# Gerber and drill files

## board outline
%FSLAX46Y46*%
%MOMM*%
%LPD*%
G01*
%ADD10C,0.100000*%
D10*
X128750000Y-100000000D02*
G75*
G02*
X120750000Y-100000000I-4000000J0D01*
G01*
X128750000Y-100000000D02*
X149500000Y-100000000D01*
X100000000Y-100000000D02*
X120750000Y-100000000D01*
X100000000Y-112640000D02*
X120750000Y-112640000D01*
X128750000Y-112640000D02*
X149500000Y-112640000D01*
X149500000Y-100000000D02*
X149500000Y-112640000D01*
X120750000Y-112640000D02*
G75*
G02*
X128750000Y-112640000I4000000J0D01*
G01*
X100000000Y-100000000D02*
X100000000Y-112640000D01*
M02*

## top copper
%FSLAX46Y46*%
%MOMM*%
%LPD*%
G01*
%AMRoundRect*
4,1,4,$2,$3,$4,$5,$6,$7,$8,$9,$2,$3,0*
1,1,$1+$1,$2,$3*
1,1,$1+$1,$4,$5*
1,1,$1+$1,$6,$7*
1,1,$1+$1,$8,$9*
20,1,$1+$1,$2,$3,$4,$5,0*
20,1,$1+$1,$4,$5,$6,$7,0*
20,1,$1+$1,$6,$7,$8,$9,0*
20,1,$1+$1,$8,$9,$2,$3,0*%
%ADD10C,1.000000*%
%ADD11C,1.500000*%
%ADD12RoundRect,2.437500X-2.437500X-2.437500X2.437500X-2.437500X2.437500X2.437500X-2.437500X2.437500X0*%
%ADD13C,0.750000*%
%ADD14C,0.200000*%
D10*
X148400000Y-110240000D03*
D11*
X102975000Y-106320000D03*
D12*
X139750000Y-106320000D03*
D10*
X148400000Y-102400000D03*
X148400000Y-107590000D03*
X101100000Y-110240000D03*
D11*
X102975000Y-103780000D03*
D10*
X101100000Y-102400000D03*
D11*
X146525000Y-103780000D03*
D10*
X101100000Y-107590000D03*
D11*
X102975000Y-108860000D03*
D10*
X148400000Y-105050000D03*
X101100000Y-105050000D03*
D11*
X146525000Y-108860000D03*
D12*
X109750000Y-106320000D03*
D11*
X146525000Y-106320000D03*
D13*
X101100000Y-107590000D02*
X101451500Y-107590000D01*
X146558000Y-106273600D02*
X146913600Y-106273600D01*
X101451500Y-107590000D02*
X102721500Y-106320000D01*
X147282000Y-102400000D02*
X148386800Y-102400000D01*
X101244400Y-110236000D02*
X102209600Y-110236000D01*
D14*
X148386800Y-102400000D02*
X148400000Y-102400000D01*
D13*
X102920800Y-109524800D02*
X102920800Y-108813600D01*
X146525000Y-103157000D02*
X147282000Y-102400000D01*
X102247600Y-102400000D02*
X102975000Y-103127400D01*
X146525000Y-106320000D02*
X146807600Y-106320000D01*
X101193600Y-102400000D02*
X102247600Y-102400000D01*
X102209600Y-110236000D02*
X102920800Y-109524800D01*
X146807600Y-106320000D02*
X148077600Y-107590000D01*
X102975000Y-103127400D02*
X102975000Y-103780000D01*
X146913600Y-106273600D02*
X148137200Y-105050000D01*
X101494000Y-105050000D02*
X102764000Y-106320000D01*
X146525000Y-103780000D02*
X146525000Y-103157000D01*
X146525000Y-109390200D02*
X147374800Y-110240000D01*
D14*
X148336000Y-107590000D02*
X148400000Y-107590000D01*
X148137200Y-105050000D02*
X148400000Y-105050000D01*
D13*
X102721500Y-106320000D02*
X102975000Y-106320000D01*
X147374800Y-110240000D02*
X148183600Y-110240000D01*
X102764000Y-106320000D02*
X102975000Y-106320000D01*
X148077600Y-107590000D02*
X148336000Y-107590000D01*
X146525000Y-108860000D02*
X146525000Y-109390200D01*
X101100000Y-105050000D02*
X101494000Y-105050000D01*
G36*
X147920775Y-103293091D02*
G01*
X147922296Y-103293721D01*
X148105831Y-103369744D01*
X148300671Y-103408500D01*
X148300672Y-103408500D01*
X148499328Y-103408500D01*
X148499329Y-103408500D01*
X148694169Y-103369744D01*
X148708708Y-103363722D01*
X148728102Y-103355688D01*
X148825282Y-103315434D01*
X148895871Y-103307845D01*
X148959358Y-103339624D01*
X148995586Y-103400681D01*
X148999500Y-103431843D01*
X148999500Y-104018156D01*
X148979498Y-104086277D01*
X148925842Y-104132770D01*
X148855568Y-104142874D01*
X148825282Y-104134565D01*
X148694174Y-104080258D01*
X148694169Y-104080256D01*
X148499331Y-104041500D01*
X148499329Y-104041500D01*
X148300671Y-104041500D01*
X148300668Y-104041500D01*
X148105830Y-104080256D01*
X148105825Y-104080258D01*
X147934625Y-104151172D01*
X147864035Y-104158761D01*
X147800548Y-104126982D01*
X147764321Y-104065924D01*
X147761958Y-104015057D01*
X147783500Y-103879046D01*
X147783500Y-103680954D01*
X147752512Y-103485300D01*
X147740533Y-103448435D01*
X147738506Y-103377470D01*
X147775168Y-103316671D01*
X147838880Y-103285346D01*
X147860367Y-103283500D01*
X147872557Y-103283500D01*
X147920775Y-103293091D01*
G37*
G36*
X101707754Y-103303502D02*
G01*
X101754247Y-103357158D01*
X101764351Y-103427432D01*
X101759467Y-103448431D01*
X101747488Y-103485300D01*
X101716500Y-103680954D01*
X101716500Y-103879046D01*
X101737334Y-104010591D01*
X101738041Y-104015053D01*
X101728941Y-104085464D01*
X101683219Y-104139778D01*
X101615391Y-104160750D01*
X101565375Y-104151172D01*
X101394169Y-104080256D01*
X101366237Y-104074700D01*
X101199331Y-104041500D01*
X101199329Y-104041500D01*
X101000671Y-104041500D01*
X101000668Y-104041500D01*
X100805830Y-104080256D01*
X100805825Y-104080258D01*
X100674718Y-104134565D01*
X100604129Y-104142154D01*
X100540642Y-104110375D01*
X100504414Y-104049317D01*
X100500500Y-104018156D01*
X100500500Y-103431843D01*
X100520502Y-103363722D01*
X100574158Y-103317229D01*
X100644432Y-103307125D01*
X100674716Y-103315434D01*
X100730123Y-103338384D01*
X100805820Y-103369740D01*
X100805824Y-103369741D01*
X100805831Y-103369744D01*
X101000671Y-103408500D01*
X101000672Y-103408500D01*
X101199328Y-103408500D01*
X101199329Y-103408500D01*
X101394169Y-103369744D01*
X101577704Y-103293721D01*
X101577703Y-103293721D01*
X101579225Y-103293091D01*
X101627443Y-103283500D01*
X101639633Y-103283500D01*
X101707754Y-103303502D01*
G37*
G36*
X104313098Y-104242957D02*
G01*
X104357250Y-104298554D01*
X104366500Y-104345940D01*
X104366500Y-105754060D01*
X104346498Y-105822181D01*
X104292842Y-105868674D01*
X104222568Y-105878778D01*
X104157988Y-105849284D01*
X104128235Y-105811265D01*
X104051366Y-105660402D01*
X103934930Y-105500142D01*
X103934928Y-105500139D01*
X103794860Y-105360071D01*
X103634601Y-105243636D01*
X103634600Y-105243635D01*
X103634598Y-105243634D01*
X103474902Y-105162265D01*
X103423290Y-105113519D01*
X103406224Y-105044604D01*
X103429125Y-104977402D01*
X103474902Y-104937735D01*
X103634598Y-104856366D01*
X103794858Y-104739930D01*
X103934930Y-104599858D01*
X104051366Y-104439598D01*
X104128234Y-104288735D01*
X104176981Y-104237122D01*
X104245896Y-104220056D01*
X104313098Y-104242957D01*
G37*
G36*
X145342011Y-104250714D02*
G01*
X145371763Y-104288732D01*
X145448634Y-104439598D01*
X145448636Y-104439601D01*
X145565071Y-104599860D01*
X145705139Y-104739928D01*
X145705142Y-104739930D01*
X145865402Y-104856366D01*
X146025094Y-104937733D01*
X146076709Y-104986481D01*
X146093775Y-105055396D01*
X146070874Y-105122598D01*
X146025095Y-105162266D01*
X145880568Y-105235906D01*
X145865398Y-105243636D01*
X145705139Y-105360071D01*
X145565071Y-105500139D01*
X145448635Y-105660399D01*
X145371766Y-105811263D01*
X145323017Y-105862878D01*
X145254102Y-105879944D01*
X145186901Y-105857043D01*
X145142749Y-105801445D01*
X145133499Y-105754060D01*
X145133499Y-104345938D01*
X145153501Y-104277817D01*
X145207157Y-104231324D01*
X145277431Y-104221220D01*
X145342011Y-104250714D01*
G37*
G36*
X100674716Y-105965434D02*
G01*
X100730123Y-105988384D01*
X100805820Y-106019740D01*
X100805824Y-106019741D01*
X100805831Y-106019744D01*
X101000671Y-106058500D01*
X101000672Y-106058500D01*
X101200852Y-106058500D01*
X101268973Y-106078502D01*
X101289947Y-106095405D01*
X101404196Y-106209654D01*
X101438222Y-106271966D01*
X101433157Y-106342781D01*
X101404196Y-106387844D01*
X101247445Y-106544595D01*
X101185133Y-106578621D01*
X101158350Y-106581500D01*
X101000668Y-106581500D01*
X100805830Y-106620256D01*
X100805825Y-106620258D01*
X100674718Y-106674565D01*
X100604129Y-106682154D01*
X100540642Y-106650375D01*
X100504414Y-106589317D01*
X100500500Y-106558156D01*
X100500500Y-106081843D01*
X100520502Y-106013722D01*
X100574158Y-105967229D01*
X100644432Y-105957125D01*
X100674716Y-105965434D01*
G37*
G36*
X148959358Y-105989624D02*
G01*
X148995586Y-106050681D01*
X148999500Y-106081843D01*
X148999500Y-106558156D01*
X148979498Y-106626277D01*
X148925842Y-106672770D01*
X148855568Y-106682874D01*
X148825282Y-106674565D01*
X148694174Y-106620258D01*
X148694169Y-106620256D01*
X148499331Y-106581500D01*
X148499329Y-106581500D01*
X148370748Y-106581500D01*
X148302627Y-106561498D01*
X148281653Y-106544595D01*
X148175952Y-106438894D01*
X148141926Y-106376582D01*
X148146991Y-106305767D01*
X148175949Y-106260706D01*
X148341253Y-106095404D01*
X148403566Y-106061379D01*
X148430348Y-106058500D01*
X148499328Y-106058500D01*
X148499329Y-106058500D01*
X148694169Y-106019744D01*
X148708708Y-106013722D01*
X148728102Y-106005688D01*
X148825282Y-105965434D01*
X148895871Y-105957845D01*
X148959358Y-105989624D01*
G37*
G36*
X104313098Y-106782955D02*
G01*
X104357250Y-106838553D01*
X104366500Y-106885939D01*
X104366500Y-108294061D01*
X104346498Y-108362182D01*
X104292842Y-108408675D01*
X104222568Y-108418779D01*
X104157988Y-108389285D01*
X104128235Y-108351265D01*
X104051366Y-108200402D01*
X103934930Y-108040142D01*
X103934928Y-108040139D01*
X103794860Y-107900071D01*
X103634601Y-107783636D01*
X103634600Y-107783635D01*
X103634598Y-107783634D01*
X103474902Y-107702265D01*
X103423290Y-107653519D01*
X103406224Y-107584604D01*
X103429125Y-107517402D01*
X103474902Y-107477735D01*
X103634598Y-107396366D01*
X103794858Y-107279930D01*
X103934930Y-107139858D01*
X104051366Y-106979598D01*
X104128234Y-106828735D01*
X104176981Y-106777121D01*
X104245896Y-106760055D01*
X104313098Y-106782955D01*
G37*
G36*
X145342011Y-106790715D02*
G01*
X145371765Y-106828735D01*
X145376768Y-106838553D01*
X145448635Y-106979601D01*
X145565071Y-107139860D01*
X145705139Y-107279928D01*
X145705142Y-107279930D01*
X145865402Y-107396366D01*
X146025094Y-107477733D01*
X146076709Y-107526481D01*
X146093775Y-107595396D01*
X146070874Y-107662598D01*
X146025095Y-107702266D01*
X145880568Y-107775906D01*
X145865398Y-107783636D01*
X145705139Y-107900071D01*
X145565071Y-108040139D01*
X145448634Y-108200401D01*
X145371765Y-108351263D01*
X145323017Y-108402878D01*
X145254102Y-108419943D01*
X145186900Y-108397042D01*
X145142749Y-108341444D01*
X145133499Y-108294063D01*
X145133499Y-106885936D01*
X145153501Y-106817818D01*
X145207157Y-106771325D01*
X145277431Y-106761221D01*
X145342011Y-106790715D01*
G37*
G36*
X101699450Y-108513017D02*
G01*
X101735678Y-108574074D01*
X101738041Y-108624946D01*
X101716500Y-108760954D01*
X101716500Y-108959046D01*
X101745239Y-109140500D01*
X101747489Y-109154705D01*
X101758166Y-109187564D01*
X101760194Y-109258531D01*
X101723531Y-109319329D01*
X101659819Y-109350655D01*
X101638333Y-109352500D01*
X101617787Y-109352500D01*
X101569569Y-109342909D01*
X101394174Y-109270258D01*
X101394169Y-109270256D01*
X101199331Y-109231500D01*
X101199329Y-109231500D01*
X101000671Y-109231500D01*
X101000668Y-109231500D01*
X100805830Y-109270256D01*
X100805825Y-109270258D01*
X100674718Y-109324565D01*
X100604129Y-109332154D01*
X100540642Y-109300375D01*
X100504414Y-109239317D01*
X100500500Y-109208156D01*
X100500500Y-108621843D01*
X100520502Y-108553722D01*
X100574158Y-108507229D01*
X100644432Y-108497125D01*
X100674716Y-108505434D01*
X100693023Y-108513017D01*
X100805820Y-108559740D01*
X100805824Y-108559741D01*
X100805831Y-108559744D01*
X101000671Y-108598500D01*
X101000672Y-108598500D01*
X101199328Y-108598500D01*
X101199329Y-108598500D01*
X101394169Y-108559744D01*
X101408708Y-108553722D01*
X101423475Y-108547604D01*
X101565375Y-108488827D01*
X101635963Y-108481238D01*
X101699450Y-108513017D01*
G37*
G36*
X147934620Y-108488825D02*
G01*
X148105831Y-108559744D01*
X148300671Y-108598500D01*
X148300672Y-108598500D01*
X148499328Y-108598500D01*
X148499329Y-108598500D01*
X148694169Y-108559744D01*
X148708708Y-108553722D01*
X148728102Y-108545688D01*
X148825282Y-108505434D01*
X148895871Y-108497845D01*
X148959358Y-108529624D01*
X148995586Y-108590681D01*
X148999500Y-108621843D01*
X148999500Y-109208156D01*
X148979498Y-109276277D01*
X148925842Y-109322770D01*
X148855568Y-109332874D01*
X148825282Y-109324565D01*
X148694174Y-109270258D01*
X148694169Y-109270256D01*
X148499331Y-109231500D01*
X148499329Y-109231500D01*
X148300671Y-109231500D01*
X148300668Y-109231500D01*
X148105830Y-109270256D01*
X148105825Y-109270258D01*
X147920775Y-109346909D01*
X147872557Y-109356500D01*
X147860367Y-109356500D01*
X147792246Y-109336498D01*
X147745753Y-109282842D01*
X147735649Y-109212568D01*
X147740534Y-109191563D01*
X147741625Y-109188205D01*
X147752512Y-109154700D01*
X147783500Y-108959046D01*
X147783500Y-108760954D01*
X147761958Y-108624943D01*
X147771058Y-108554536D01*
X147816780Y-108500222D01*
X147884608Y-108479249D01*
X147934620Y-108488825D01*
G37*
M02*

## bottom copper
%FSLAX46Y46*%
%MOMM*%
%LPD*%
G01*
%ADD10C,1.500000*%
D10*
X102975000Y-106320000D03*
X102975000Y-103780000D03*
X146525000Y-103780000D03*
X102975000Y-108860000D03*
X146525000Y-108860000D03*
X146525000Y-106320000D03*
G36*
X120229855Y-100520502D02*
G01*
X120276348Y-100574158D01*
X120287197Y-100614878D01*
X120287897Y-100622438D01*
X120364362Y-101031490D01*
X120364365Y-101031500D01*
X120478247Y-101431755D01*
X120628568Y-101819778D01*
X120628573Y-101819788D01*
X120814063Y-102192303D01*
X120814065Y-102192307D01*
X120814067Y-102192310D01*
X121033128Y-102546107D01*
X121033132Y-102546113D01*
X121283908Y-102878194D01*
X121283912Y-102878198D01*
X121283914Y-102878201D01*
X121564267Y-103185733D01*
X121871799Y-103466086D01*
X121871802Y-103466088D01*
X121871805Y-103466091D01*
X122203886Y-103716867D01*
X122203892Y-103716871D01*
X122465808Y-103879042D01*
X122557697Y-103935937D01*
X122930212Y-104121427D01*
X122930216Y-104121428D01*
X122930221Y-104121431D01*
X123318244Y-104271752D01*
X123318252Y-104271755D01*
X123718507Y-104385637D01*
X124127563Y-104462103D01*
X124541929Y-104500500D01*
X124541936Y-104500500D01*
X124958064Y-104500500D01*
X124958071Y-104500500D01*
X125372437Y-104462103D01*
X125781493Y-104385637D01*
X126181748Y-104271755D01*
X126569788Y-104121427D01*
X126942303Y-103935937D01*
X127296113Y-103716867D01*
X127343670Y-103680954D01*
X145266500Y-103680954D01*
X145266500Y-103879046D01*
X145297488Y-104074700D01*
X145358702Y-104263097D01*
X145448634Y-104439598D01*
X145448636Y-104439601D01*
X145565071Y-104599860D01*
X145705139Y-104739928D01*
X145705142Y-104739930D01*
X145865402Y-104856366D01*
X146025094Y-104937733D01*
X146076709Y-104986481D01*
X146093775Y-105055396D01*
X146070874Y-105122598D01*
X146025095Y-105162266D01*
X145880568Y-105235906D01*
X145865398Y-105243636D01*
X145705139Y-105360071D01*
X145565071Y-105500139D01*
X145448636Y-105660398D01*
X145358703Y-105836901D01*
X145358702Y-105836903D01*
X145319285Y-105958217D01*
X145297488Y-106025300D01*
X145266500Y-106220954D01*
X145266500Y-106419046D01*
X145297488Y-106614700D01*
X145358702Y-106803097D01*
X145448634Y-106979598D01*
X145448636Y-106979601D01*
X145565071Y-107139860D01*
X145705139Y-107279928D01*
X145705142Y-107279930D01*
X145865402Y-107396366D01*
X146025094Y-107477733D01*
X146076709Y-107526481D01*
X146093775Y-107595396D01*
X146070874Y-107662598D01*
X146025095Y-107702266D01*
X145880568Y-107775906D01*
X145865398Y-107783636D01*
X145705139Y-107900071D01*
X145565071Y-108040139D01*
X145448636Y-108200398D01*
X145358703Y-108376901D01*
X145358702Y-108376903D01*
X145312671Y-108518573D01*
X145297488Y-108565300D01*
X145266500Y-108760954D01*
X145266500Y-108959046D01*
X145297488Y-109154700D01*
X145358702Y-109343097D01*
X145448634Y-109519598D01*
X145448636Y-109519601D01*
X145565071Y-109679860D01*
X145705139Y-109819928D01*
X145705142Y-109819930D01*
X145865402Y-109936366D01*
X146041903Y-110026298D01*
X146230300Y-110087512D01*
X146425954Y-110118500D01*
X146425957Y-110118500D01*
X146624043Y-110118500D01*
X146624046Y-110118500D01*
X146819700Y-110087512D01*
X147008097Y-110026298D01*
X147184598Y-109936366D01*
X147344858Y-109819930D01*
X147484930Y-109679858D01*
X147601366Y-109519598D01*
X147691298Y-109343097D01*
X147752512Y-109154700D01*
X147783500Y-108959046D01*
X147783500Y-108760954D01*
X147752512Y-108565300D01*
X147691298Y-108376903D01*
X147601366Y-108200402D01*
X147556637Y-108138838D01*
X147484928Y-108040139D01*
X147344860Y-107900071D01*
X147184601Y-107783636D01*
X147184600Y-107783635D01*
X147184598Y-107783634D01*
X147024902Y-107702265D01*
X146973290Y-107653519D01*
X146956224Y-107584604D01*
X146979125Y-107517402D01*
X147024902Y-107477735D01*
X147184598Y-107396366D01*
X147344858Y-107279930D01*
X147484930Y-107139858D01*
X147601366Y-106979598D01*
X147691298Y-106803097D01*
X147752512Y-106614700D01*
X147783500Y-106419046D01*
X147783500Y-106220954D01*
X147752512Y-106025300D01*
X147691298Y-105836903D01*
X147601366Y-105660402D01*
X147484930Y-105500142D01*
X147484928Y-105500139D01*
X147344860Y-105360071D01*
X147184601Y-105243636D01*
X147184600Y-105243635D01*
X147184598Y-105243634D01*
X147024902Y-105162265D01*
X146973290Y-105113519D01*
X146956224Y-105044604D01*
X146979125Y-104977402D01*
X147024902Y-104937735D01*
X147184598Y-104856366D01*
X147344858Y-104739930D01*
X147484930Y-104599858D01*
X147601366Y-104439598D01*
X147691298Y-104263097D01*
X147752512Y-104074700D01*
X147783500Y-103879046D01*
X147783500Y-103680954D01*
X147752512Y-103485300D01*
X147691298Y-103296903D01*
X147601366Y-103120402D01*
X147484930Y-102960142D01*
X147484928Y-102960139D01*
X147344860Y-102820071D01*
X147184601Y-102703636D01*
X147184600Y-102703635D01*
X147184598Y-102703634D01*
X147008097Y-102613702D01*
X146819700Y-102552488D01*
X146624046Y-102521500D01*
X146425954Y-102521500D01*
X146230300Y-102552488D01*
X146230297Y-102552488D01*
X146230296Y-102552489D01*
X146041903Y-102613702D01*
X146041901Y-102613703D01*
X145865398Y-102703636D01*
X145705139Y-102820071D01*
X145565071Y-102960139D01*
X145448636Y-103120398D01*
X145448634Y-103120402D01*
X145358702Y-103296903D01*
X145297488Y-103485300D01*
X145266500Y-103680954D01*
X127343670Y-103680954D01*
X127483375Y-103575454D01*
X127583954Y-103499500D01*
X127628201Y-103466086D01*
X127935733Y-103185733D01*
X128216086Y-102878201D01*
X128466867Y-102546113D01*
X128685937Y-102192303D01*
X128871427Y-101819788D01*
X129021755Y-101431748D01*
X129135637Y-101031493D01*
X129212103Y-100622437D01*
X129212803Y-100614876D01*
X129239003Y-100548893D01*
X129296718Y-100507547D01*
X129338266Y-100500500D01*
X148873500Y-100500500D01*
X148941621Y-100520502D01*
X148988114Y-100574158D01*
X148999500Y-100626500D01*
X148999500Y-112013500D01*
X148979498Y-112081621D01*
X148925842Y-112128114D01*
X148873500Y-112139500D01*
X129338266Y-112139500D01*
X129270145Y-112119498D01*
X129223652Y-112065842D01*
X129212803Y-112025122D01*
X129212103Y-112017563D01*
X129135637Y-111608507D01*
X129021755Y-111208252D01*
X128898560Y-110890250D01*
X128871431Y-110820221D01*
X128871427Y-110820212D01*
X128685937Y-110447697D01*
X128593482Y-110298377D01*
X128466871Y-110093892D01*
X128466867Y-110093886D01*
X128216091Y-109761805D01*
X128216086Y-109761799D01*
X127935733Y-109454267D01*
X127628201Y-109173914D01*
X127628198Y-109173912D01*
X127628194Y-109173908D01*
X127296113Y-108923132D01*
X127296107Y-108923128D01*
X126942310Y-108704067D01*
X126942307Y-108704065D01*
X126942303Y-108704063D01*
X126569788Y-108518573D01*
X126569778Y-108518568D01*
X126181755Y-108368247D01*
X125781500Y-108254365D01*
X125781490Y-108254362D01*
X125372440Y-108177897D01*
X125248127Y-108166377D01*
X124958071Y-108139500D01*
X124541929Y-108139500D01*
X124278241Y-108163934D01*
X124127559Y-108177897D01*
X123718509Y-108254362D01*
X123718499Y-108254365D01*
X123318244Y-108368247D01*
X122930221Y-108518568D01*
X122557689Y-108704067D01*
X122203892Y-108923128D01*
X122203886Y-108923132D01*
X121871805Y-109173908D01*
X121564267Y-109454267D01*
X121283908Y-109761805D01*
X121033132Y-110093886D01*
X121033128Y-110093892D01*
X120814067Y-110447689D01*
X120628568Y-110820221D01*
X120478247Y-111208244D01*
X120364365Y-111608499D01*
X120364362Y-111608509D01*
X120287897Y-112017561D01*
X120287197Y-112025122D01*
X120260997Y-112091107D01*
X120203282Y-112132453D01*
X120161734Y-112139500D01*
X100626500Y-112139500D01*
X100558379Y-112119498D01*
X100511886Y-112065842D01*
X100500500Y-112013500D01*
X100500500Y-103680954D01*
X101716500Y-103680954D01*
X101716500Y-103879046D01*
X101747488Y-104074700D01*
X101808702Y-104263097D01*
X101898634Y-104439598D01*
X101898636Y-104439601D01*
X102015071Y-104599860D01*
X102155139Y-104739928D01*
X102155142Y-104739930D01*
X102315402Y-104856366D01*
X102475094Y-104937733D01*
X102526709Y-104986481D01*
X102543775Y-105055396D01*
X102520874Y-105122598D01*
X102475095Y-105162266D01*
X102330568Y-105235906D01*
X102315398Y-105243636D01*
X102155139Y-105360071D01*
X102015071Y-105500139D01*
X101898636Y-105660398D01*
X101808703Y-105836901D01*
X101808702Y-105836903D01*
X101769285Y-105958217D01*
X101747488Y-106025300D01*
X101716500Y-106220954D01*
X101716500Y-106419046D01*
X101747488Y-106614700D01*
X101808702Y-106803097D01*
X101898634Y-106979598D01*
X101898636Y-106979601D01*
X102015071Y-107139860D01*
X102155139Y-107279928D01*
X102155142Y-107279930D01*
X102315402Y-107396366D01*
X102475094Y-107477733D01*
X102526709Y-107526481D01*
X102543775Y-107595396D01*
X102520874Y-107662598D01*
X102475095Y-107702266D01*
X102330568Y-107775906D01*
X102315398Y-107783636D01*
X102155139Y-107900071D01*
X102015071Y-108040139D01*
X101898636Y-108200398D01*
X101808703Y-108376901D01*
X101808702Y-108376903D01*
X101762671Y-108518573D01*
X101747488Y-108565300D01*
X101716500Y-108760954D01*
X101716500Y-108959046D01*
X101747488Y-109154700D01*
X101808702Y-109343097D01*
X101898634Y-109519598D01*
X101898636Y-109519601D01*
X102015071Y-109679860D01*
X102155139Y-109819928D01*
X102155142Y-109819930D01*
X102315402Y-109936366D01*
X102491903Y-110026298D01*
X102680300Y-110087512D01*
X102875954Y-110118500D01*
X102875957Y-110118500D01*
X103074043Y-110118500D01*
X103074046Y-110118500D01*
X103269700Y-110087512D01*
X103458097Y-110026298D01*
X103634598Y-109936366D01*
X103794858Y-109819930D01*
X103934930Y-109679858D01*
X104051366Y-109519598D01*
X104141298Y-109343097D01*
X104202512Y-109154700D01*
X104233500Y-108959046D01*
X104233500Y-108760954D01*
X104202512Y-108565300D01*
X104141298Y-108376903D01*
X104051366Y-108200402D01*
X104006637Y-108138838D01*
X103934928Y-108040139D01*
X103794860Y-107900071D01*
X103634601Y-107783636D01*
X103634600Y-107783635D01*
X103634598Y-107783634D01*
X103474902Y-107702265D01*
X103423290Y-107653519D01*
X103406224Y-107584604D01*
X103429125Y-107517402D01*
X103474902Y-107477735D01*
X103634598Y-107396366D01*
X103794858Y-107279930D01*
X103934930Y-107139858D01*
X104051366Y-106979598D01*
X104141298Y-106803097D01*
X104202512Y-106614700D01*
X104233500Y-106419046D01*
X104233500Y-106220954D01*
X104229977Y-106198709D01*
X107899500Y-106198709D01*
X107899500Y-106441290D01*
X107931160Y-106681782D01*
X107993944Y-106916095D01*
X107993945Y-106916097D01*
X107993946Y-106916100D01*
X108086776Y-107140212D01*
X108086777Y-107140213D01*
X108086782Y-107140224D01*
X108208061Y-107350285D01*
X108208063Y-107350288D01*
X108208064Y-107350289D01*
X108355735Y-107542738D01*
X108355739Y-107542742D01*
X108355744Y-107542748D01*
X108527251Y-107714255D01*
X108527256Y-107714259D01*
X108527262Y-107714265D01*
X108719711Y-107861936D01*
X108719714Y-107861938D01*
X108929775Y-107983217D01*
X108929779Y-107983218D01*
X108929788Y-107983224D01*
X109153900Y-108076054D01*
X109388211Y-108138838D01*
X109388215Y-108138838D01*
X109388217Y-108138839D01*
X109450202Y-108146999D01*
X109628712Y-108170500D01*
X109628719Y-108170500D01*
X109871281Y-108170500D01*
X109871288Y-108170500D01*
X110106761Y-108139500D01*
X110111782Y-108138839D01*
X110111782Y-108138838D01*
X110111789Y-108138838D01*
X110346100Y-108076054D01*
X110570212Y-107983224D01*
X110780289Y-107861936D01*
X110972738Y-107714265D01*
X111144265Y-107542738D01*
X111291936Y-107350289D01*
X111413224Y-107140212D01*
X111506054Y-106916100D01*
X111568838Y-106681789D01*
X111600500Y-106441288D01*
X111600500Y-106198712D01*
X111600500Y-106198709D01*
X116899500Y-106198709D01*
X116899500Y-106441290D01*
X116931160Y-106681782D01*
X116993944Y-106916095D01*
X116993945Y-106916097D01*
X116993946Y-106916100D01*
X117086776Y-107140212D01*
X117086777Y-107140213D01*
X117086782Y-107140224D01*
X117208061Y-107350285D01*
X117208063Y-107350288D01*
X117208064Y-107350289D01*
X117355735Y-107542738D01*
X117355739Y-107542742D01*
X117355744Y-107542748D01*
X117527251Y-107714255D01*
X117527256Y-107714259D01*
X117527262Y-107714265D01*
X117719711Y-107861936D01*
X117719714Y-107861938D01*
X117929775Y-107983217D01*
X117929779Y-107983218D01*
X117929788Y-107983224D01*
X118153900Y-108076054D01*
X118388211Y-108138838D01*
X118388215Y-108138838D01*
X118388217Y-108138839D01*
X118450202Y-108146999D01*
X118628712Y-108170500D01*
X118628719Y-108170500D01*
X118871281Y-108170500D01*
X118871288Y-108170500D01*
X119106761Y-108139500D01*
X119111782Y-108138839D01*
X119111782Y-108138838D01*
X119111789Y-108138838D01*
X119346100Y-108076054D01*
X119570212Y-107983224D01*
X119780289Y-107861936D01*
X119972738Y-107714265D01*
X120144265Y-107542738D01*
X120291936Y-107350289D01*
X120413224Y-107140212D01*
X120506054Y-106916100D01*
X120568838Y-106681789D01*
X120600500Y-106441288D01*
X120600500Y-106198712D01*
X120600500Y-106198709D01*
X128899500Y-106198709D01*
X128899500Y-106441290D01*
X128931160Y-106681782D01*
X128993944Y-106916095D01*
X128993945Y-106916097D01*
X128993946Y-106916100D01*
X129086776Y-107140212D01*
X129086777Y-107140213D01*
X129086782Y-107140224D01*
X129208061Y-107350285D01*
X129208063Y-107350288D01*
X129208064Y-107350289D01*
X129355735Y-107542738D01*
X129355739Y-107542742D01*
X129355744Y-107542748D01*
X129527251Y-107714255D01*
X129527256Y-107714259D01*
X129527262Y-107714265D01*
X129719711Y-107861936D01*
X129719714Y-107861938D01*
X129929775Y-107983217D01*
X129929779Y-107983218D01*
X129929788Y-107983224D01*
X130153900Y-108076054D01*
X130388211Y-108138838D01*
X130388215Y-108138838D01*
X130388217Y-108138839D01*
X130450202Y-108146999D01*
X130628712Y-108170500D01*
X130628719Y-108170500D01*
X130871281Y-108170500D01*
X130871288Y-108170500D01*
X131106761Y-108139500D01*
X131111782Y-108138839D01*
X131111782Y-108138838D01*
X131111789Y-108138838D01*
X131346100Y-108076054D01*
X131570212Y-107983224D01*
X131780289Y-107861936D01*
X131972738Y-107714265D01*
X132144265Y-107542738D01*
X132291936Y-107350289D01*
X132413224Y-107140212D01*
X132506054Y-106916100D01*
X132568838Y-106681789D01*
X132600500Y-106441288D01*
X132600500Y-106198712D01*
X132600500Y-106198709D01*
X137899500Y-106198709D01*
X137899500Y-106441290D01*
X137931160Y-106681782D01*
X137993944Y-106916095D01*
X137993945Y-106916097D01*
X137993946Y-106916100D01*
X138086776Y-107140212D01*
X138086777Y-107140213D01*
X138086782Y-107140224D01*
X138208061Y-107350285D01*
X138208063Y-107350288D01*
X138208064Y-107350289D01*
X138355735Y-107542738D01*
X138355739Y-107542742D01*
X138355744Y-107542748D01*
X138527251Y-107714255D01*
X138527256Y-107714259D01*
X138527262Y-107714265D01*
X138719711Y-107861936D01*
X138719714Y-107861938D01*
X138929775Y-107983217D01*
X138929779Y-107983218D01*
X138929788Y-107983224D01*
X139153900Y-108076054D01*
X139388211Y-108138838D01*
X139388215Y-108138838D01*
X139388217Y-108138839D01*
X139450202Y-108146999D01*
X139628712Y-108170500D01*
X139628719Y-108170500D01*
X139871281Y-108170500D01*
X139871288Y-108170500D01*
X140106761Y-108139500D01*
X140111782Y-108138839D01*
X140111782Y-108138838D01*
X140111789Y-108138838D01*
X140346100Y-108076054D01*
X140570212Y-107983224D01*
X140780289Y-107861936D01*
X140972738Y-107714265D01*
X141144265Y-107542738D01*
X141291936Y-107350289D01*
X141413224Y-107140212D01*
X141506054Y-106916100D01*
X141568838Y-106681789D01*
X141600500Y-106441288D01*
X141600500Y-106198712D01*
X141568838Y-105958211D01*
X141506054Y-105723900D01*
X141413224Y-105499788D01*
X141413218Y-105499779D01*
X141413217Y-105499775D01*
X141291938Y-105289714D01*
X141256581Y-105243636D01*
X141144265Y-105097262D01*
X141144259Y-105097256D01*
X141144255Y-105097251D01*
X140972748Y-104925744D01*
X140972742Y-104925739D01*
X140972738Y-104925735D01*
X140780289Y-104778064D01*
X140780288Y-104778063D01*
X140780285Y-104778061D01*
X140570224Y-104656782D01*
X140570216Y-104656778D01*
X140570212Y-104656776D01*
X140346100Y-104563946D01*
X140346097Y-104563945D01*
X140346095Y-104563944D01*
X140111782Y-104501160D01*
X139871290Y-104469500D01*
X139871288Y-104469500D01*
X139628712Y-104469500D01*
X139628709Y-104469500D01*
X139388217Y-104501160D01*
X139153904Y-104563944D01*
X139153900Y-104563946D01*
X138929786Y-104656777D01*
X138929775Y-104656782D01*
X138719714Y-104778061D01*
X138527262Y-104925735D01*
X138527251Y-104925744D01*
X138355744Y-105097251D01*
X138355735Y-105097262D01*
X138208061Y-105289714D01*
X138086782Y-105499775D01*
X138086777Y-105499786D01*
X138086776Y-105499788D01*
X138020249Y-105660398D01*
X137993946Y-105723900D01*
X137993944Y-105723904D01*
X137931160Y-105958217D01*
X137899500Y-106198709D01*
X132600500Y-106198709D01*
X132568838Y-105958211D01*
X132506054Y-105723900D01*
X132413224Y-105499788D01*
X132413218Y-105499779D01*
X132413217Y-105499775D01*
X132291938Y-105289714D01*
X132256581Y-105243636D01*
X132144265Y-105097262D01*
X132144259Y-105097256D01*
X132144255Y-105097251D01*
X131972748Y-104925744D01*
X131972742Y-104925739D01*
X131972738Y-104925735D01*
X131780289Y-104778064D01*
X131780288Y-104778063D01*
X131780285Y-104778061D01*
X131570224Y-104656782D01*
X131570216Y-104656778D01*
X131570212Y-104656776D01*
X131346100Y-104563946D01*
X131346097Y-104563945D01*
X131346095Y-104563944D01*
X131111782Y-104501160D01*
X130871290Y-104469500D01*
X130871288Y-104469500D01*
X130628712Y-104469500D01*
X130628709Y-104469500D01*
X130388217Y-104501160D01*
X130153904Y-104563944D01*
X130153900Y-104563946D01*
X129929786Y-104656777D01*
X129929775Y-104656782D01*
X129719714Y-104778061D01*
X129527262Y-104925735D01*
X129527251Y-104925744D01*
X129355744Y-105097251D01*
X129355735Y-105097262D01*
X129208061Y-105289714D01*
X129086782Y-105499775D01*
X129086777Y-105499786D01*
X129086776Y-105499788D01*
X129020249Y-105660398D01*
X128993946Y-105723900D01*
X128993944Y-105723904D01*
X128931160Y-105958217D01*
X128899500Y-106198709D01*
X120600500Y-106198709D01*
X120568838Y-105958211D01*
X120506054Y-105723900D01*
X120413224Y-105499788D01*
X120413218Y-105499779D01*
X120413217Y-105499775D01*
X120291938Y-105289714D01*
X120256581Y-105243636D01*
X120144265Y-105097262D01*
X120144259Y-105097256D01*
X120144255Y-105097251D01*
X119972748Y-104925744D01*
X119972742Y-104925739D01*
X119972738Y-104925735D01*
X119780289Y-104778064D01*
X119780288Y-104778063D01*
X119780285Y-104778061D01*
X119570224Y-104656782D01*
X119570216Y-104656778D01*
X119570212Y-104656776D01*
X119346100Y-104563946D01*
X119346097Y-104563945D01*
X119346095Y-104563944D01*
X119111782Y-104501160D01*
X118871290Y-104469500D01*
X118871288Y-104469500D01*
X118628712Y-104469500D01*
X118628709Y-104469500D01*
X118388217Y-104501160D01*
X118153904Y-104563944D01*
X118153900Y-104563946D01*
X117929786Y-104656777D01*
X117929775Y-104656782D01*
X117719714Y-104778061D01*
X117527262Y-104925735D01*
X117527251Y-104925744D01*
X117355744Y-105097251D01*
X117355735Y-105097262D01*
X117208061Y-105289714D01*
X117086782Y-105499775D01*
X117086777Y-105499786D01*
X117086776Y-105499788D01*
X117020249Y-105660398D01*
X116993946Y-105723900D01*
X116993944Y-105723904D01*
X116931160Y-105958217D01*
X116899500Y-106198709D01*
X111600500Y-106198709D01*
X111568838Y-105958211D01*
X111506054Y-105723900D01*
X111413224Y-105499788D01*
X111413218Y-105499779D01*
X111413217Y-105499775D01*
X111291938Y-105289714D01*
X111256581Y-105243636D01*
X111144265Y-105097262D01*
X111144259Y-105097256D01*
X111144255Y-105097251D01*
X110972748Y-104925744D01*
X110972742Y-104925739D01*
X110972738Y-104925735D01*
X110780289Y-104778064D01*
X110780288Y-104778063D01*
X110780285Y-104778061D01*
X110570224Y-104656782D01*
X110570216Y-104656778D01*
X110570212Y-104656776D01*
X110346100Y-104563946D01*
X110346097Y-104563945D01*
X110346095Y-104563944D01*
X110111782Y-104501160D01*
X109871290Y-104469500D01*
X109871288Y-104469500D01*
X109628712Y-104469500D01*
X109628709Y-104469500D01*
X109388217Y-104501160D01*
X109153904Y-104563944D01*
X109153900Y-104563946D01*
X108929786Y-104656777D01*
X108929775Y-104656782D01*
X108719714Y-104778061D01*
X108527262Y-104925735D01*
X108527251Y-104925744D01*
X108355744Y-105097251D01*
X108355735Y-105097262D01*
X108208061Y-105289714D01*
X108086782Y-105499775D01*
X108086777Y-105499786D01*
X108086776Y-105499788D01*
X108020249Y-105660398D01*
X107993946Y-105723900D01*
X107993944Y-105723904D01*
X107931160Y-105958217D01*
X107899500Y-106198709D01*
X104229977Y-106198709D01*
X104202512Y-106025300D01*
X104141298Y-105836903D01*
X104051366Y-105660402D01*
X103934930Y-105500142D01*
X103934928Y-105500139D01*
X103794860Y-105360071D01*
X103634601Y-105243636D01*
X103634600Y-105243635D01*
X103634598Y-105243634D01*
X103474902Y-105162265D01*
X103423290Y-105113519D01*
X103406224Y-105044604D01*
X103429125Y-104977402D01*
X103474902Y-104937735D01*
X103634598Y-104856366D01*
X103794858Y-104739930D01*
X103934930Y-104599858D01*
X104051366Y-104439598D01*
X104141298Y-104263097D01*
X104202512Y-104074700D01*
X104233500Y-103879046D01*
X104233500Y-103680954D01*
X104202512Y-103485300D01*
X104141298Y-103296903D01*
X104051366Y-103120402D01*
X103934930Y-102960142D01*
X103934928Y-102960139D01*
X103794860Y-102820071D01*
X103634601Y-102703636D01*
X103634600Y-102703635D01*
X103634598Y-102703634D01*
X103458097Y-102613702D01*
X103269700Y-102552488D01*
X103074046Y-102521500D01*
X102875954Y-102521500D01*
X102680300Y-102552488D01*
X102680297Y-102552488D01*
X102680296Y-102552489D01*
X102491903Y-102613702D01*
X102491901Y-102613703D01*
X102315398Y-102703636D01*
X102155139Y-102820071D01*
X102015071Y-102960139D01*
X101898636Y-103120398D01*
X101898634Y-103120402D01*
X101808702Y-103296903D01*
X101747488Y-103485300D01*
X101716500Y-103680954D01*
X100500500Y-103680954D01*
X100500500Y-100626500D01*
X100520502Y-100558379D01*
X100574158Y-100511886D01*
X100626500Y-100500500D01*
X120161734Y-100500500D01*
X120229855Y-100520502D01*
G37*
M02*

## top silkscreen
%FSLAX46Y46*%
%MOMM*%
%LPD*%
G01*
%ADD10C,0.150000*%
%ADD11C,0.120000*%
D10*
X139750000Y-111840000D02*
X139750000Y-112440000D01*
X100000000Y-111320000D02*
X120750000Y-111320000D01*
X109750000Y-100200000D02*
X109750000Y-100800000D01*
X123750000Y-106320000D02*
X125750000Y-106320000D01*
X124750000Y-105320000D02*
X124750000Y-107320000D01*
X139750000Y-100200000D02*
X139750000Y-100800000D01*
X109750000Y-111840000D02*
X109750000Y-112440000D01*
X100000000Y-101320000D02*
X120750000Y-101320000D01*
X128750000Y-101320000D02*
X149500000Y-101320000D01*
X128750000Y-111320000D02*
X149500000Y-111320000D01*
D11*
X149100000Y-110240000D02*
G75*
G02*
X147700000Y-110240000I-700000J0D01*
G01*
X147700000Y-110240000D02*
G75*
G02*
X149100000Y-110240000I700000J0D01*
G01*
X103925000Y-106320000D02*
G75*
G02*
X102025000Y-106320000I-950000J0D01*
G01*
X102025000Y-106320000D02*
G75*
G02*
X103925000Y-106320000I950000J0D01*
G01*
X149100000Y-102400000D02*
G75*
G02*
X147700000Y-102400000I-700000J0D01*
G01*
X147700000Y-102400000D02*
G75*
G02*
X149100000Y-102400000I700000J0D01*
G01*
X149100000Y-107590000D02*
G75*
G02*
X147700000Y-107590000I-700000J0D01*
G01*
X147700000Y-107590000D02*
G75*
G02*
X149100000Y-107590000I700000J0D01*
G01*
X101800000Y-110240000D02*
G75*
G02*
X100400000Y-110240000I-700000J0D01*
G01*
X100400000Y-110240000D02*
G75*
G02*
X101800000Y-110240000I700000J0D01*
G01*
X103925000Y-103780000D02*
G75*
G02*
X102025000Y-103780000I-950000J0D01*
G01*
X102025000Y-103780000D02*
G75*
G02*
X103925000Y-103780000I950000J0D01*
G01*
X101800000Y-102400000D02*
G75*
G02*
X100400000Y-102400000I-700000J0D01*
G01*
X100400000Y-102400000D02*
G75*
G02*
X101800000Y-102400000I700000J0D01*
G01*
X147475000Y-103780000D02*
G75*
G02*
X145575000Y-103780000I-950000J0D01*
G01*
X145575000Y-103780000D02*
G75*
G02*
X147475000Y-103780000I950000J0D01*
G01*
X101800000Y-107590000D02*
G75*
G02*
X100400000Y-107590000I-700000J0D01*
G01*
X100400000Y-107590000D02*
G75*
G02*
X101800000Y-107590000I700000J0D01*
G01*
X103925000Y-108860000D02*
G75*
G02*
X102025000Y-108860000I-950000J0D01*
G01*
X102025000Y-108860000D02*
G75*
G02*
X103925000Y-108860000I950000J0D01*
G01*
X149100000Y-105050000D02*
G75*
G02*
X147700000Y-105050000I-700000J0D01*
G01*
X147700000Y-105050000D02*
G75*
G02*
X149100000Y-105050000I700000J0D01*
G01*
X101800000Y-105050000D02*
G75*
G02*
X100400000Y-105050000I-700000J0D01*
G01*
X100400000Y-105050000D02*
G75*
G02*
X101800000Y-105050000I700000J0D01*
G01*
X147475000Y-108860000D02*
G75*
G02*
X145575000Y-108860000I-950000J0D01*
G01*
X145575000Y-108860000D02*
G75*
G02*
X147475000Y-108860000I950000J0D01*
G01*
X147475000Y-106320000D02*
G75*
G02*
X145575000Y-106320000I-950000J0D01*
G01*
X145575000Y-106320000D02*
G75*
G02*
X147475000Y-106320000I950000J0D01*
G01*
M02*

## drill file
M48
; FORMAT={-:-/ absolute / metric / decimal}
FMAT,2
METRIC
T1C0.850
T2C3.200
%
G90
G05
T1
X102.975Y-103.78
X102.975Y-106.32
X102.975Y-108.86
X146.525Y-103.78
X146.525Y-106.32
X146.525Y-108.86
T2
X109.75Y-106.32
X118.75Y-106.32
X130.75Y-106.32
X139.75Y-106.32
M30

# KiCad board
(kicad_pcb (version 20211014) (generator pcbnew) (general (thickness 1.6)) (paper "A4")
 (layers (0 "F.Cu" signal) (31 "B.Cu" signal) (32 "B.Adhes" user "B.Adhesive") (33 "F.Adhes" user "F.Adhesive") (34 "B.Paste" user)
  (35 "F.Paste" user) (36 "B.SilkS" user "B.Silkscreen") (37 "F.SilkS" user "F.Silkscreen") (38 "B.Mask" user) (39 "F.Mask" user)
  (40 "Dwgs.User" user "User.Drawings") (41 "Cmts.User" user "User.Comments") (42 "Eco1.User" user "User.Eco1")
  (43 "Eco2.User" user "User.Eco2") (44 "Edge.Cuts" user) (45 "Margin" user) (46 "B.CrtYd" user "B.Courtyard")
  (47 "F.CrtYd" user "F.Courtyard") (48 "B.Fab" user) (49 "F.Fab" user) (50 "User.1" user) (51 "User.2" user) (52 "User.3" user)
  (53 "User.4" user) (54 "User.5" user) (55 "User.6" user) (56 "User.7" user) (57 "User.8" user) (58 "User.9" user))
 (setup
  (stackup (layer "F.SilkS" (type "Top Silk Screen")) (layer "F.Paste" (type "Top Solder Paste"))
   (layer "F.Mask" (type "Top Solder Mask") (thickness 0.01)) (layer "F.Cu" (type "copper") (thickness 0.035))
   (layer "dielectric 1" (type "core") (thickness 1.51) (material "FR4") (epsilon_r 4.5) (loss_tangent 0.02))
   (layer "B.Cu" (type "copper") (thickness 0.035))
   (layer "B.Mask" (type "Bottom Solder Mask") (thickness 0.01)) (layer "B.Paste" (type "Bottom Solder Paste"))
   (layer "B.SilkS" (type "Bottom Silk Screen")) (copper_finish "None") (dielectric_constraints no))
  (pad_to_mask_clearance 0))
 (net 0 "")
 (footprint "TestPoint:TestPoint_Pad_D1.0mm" (layer "F.Cu") (at 148.4 110.24)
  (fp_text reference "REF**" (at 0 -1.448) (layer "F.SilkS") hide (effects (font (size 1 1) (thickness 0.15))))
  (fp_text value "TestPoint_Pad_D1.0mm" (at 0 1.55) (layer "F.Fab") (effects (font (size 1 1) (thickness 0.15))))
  (fp_circle (center 0 0) (end 0 0.7) (layer "F.SilkS") (width 0.12) (fill none))
  (pad "1" smd circle (at 0 0) (size 1 1) (layers "F.Cu" "F.Mask")))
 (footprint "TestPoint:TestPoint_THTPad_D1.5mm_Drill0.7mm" (layer "F.Cu") (at 102.975 106.32)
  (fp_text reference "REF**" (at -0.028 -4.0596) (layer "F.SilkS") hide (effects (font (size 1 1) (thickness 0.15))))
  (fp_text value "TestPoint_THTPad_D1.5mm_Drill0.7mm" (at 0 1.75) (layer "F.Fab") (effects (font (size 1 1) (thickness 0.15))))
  (fp_circle (center 0 0) (end 0 0.95) (layer "F.SilkS") (width 0.12) (fill none))
  (pad "1" thru_hole circle (at 0 0) (size 1.5 1.5) (drill 0.85) (layers *.Cu *.Mask)))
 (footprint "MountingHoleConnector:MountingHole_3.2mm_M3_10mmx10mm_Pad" (layer "F.Cu") (at 139.75 106.32)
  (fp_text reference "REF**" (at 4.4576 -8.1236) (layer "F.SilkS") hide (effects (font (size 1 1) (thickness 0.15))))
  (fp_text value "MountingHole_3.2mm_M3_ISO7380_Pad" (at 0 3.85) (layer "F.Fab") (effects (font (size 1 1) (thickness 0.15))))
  (pad "" np_thru_hole roundrect (at 0 0) (size 9.75 9.75) (drill 3.2) (layers "F.Cu" "F.Mask") (roundrect_rratio 0.25)))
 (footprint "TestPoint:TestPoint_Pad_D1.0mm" (layer "F.Cu") (at 148.4 102.4)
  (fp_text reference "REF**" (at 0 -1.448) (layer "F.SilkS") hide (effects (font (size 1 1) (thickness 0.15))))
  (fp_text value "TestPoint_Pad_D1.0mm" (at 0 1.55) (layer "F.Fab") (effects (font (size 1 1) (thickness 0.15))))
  (fp_circle (center 0 0) (end 0 0.7) (layer "F.SilkS") (width 0.12) (fill none))
  (pad "1" smd circle (at 0 0) (size 1 1) (layers "F.Cu" "F.Mask")))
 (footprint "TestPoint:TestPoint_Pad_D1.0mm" (layer "F.Cu") (at 148.4 107.59)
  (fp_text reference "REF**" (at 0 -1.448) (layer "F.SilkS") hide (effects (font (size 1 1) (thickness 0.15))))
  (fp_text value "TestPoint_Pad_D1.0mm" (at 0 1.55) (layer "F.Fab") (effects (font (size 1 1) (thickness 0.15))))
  (fp_circle (center 0 0) (end 0 0.7) (layer "F.SilkS") (width 0.12) (fill none))
  (pad "1" smd circle (at 0 0) (size 1 1) (layers "F.Cu" "F.Mask")))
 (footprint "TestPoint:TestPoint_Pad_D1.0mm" (layer "F.Cu") (at 101.1 110.24)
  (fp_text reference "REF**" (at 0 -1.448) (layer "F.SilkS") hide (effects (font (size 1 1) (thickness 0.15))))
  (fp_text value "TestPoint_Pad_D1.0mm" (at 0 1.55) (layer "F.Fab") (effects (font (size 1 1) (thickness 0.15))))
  (fp_circle (center 0 0) (end 0 0.7) (layer "F.SilkS") (width 0.12) (fill none))
  (pad "1" smd circle (at 0 0) (size 1 1) (layers "F.Cu" "F.Mask")))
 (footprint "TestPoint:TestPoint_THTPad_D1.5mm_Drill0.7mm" (layer "F.Cu") (at 102.975 103.78)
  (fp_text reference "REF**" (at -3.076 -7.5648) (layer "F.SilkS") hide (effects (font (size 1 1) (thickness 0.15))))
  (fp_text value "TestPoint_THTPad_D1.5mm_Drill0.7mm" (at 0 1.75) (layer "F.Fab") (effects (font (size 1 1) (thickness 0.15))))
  (fp_circle (center 0 0) (end 0 0.95) (layer "F.SilkS") (width 0.12) (fill none))
  (pad "1" thru_hole circle (at 0 0) (size 1.5 1.5) (drill 0.85) (layers *.Cu *.Mask)))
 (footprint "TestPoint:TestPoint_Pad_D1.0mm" (layer "F.Cu") (at 101.1 102.4)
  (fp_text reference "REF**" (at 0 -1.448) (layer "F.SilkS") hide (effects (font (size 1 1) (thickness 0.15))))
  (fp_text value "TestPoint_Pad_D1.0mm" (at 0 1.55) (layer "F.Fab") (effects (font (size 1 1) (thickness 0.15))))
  (fp_circle (center 0 0) (end 0 0.7) (layer "F.SilkS") (width 0.12) (fill none))
  (pad "1" smd circle (at 0 0) (size 1 1) (layers "F.Cu" "F.Mask")))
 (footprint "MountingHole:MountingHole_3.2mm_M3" (layer "F.Cu") (at 130.75 106.32)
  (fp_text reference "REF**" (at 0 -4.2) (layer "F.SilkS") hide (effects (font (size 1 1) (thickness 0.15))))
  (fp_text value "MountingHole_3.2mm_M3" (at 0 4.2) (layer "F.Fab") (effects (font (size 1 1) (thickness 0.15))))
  (pad "" np_thru_hole circle (at 0 0) (size 3.2 3.2) (drill 3.2) (layers *.Cu *.Mask)))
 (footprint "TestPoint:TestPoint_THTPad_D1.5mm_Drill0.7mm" (layer "F.Cu") (at 146.525 103.78)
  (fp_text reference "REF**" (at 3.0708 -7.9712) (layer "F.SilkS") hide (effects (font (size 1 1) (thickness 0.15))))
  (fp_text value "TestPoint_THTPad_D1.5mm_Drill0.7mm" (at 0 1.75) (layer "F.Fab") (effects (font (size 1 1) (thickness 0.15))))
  (fp_circle (center 0 0) (end 0 0.95) (layer "F.SilkS") (width 0.12) (fill none))
  (pad "1" thru_hole circle (at 0 0) (size 1.5 1.5) (drill 0.85) (layers *.Cu *.Mask)))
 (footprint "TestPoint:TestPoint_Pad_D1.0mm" (layer "F.Cu") (at 101.1 107.59)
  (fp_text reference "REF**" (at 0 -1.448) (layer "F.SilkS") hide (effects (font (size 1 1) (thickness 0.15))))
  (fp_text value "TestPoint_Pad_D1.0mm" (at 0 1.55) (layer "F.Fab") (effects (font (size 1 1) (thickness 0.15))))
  (fp_circle (center 0 0) (end 0 0.7) (layer "F.SilkS") (width 0.12) (fill none))
  (pad "1" smd circle (at 0 0) (size 1 1) (layers "F.Cu" "F.Mask")))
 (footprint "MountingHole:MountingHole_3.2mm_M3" (layer "F.Cu") (at 118.75 106.32)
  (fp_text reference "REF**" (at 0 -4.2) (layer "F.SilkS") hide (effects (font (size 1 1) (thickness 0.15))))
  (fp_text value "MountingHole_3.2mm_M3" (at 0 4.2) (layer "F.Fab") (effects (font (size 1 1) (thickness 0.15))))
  (pad "" np_thru_hole circle (at 0 0) (size 3.2 3.2) (drill 3.2) (layers *.Cu *.Mask)))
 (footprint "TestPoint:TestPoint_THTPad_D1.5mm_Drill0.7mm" (layer "F.Cu") (at 102.975 108.86)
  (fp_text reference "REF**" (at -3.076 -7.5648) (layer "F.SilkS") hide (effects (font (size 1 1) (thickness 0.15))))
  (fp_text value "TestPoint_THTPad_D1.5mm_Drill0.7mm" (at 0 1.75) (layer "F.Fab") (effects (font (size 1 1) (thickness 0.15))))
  (fp_circle (center 0 0) (end 0 0.95) (layer "F.SilkS") (width 0.12) (fill none))
  (pad "1" thru_hole circle (at 0 0) (size 1.5 1.5) (drill 0.85) (layers *.Cu *.Mask)))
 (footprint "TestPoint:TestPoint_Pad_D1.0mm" (layer "F.Cu") (at 148.4 105.05)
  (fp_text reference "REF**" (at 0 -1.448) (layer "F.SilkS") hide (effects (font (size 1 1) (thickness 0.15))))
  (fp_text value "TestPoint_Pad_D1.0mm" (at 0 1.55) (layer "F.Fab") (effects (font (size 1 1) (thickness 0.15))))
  (fp_circle (center 0 0) (end 0 0.7) (layer "F.SilkS") (width 0.12) (fill none))
  (pad "1" smd circle (at 0 0) (size 1 1) (layers "F.Cu" "F.Mask")))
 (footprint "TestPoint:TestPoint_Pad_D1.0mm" (layer "F.Cu") (at 101.1 105.05)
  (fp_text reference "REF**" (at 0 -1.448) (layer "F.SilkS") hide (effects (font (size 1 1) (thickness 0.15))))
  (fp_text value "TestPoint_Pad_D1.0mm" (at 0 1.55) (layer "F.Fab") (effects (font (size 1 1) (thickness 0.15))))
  (fp_circle (center 0 0) (end 0 0.7) (layer "F.SilkS") (width 0.12) (fill none))
  (pad "1" smd circle (at 0 0) (size 1 1) (layers "F.Cu" "F.Mask")))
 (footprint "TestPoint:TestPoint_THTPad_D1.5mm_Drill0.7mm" (layer "F.Cu") (at 146.525 108.86)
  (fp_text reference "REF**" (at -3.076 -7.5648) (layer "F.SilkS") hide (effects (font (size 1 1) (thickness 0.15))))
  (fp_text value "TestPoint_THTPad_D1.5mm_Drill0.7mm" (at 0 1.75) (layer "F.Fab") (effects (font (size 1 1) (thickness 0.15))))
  (fp_circle (center 0 0) (end 0 0.95) (layer "F.SilkS") (width 0.12) (fill none))
  (pad "1" thru_hole circle (at 0 0) (size 1.5 1.5) (drill 0.85) (layers *.Cu *.Mask)))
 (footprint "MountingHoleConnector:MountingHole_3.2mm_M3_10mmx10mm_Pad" (layer "F.Cu") (at 109.75 106.32)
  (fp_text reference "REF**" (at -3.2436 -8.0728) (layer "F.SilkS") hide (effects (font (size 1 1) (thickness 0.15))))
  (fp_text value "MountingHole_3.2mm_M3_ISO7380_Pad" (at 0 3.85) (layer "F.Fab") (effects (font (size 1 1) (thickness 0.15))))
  (pad "" np_thru_hole roundrect (at 0 0) (size 9.75 9.75) (drill 3.2) (layers "F.Cu" "F.Mask") (roundrect_rratio 0.25)))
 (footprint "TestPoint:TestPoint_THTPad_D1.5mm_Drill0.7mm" (layer "F.Cu") (at 146.525 106.32)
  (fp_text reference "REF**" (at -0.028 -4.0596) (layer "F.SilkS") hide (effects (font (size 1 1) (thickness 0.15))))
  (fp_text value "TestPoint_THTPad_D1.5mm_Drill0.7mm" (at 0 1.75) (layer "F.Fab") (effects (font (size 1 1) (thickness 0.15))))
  (fp_circle (center 0 0) (end 0 0.95) (layer "F.SilkS") (width 0.12) (fill none))
  (pad "1" thru_hole circle (at 0 0) (size 1.5 1.5) (drill 0.85) (layers *.Cu *.Mask)))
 (gr_line (start 139.75 111.84) (end 139.75 112.44) (layer "F.SilkS") (width 0.15))
 (gr_line (start 100 111.32) (end 120.75 111.32) (layer "F.SilkS") (width 0.15))
 (gr_line (start 109.75 100.2) (end 109.75 100.8) (layer "F.SilkS") (width 0.15))
 (gr_line (start 123.75 106.32) (end 125.75 106.32) (layer "F.SilkS") (width 0.15))
 (gr_line (start 124.75 105.32) (end 124.75 107.32) (layer "F.SilkS") (width 0.15))
 (gr_line (start 139.75 100.2) (end 139.75 100.8) (layer "F.SilkS") (width 0.15))
 (gr_line (start 109.75 111.84) (end 109.75 112.44) (layer "F.SilkS") (width 0.15))
 (gr_line (start 100 101.32) (end 120.75 101.32) (layer "F.SilkS") (width 0.15))
 (gr_line (start 128.75 101.32) (end 149.5 101.32) (layer "F.SilkS") (width 0.15))
 (gr_line (start 128.75 111.32) (end 149.5 111.32) (layer "F.SilkS") (width 0.15))
 (gr_arc (start 128.75 100) (mid 124.75 104) (end 120.75 100) (layer "Edge.Cuts") (width 0.1))
 (gr_line (start 128.75 100) (end 149.5 100) (layer "Edge.Cuts") (width 0.1))
 (gr_line (start 100 100) (end 120.75 100) (layer "Edge.Cuts") (width 0.1))
 (gr_line (start 100 112.64) (end 120.75 112.64) (layer "Edge.Cuts") (width 0.1))
 (gr_line (start 128.75 112.64) (end 149.5 112.64) (layer "Edge.Cuts") (width 0.1))
 (gr_line (start 149.5 100) (end 149.5 112.64) (layer "Edge.Cuts") (width 0.1))
 (gr_arc (start 120.75 112.64) (mid 124.75 108.64) (end 128.75 112.64) (layer "Edge.Cuts") (width 0.1))
 (gr_line (start 100 100) (end 100 112.64) (layer "Edge.Cuts") (width 0.1))
 (segment (start 101.1 107.59) (end 101.4515 107.59) (width 0.75) (layer "F.Cu") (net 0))
 (segment (start 146.558 106.2736) (end 146.9136 106.2736) (width 0.75) (layer "F.Cu") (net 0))
 (segment (start 101.4515 107.59) (end 102.7215 106.32) (width 0.75) (layer "F.Cu") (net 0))
 (segment (start 147.282 102.4) (end 148.3868 102.4) (width 0.75) (layer "F.Cu") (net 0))
 (segment (start 101.2444 110.236) (end 102.2096 110.236) (width 0.75) (layer "F.Cu") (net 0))
 (segment (start 148.3868 102.4) (end 148.4 102.4) (width 0.2) (layer "F.Cu") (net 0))
 (segment (start 102.9208 109.5248) (end 102.9208 108.8136) (width 0.75) (layer "F.Cu") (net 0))
 (segment (start 146.525 103.157) (end 147.282 102.4) (width 0.75) (layer "F.Cu") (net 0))
 (segment (start 102.2476 102.4) (end 102.975 103.1274) (width 0.75) (layer "F.Cu") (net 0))
 (segment (start 146.525 106.32) (end 146.8076 106.32) (width 0.75) (layer "F.Cu") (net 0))
 (segment (start 101.1936 102.4) (end 102.2476 102.4) (width 0.75) (layer "F.Cu") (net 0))
 (segment (start 102.2096 110.236) (end 102.9208 109.5248) (width 0.75) (layer "F.Cu") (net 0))
 (segment (start 146.8076 106.32) (end 148.0776 107.59) (width 0.75) (layer "F.Cu") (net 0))
 (segment (start 102.975 103.1274) (end 102.975 103.78) (width 0.75) (layer "F.Cu") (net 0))
 (segment (start 146.9136 106.2736) (end 148.1372 105.05) (width 0.75) (layer "F.Cu") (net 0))
 (segment (start 101.494 105.05) (end 102.764 106.32) (width 0.75) (layer "F.Cu") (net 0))
 (segment (start 146.525 103.78) (end 146.525 103.157) (width 0.75) (layer "F.Cu") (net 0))
 (segment (start 146.525 109.3902) (end 147.3748 110.24) (width 0.75) (layer "F.Cu") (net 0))
 (segment (start 148.336 107.59) (end 148.4 107.59) (width 0.2) (layer "F.Cu") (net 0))
 (segment (start 148.1372 105.05) (end 148.4 105.05) (width 0.2) (layer "F.Cu") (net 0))
 (segment (start 102.7215 106.32) (end 102.975 106.32) (width 0.75) (layer "F.Cu") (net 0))
 (segment (start 147.3748 110.24) (end 148.1836 110.24) (width 0.75) (layer "F.Cu") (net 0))
 (segment (start 102.764 106.32) (end 102.975 106.32) (width 0.75) (layer "F.Cu") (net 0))
 (segment (start 148.0776 107.59) (end 148.336 107.59) (width 0.75) (layer "F.Cu") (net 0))
 (segment (start 146.525 108.86) (end 146.525 109.3902) (width 0.75) (layer "F.Cu") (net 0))
 (segment (start 101.1 105.05) (end 101.494 105.05) (width 0.75) (layer "F.Cu") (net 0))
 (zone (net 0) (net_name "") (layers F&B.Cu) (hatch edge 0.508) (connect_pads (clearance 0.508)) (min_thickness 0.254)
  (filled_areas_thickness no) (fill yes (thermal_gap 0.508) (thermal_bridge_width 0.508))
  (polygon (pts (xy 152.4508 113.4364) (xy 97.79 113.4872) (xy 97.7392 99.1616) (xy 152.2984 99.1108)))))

